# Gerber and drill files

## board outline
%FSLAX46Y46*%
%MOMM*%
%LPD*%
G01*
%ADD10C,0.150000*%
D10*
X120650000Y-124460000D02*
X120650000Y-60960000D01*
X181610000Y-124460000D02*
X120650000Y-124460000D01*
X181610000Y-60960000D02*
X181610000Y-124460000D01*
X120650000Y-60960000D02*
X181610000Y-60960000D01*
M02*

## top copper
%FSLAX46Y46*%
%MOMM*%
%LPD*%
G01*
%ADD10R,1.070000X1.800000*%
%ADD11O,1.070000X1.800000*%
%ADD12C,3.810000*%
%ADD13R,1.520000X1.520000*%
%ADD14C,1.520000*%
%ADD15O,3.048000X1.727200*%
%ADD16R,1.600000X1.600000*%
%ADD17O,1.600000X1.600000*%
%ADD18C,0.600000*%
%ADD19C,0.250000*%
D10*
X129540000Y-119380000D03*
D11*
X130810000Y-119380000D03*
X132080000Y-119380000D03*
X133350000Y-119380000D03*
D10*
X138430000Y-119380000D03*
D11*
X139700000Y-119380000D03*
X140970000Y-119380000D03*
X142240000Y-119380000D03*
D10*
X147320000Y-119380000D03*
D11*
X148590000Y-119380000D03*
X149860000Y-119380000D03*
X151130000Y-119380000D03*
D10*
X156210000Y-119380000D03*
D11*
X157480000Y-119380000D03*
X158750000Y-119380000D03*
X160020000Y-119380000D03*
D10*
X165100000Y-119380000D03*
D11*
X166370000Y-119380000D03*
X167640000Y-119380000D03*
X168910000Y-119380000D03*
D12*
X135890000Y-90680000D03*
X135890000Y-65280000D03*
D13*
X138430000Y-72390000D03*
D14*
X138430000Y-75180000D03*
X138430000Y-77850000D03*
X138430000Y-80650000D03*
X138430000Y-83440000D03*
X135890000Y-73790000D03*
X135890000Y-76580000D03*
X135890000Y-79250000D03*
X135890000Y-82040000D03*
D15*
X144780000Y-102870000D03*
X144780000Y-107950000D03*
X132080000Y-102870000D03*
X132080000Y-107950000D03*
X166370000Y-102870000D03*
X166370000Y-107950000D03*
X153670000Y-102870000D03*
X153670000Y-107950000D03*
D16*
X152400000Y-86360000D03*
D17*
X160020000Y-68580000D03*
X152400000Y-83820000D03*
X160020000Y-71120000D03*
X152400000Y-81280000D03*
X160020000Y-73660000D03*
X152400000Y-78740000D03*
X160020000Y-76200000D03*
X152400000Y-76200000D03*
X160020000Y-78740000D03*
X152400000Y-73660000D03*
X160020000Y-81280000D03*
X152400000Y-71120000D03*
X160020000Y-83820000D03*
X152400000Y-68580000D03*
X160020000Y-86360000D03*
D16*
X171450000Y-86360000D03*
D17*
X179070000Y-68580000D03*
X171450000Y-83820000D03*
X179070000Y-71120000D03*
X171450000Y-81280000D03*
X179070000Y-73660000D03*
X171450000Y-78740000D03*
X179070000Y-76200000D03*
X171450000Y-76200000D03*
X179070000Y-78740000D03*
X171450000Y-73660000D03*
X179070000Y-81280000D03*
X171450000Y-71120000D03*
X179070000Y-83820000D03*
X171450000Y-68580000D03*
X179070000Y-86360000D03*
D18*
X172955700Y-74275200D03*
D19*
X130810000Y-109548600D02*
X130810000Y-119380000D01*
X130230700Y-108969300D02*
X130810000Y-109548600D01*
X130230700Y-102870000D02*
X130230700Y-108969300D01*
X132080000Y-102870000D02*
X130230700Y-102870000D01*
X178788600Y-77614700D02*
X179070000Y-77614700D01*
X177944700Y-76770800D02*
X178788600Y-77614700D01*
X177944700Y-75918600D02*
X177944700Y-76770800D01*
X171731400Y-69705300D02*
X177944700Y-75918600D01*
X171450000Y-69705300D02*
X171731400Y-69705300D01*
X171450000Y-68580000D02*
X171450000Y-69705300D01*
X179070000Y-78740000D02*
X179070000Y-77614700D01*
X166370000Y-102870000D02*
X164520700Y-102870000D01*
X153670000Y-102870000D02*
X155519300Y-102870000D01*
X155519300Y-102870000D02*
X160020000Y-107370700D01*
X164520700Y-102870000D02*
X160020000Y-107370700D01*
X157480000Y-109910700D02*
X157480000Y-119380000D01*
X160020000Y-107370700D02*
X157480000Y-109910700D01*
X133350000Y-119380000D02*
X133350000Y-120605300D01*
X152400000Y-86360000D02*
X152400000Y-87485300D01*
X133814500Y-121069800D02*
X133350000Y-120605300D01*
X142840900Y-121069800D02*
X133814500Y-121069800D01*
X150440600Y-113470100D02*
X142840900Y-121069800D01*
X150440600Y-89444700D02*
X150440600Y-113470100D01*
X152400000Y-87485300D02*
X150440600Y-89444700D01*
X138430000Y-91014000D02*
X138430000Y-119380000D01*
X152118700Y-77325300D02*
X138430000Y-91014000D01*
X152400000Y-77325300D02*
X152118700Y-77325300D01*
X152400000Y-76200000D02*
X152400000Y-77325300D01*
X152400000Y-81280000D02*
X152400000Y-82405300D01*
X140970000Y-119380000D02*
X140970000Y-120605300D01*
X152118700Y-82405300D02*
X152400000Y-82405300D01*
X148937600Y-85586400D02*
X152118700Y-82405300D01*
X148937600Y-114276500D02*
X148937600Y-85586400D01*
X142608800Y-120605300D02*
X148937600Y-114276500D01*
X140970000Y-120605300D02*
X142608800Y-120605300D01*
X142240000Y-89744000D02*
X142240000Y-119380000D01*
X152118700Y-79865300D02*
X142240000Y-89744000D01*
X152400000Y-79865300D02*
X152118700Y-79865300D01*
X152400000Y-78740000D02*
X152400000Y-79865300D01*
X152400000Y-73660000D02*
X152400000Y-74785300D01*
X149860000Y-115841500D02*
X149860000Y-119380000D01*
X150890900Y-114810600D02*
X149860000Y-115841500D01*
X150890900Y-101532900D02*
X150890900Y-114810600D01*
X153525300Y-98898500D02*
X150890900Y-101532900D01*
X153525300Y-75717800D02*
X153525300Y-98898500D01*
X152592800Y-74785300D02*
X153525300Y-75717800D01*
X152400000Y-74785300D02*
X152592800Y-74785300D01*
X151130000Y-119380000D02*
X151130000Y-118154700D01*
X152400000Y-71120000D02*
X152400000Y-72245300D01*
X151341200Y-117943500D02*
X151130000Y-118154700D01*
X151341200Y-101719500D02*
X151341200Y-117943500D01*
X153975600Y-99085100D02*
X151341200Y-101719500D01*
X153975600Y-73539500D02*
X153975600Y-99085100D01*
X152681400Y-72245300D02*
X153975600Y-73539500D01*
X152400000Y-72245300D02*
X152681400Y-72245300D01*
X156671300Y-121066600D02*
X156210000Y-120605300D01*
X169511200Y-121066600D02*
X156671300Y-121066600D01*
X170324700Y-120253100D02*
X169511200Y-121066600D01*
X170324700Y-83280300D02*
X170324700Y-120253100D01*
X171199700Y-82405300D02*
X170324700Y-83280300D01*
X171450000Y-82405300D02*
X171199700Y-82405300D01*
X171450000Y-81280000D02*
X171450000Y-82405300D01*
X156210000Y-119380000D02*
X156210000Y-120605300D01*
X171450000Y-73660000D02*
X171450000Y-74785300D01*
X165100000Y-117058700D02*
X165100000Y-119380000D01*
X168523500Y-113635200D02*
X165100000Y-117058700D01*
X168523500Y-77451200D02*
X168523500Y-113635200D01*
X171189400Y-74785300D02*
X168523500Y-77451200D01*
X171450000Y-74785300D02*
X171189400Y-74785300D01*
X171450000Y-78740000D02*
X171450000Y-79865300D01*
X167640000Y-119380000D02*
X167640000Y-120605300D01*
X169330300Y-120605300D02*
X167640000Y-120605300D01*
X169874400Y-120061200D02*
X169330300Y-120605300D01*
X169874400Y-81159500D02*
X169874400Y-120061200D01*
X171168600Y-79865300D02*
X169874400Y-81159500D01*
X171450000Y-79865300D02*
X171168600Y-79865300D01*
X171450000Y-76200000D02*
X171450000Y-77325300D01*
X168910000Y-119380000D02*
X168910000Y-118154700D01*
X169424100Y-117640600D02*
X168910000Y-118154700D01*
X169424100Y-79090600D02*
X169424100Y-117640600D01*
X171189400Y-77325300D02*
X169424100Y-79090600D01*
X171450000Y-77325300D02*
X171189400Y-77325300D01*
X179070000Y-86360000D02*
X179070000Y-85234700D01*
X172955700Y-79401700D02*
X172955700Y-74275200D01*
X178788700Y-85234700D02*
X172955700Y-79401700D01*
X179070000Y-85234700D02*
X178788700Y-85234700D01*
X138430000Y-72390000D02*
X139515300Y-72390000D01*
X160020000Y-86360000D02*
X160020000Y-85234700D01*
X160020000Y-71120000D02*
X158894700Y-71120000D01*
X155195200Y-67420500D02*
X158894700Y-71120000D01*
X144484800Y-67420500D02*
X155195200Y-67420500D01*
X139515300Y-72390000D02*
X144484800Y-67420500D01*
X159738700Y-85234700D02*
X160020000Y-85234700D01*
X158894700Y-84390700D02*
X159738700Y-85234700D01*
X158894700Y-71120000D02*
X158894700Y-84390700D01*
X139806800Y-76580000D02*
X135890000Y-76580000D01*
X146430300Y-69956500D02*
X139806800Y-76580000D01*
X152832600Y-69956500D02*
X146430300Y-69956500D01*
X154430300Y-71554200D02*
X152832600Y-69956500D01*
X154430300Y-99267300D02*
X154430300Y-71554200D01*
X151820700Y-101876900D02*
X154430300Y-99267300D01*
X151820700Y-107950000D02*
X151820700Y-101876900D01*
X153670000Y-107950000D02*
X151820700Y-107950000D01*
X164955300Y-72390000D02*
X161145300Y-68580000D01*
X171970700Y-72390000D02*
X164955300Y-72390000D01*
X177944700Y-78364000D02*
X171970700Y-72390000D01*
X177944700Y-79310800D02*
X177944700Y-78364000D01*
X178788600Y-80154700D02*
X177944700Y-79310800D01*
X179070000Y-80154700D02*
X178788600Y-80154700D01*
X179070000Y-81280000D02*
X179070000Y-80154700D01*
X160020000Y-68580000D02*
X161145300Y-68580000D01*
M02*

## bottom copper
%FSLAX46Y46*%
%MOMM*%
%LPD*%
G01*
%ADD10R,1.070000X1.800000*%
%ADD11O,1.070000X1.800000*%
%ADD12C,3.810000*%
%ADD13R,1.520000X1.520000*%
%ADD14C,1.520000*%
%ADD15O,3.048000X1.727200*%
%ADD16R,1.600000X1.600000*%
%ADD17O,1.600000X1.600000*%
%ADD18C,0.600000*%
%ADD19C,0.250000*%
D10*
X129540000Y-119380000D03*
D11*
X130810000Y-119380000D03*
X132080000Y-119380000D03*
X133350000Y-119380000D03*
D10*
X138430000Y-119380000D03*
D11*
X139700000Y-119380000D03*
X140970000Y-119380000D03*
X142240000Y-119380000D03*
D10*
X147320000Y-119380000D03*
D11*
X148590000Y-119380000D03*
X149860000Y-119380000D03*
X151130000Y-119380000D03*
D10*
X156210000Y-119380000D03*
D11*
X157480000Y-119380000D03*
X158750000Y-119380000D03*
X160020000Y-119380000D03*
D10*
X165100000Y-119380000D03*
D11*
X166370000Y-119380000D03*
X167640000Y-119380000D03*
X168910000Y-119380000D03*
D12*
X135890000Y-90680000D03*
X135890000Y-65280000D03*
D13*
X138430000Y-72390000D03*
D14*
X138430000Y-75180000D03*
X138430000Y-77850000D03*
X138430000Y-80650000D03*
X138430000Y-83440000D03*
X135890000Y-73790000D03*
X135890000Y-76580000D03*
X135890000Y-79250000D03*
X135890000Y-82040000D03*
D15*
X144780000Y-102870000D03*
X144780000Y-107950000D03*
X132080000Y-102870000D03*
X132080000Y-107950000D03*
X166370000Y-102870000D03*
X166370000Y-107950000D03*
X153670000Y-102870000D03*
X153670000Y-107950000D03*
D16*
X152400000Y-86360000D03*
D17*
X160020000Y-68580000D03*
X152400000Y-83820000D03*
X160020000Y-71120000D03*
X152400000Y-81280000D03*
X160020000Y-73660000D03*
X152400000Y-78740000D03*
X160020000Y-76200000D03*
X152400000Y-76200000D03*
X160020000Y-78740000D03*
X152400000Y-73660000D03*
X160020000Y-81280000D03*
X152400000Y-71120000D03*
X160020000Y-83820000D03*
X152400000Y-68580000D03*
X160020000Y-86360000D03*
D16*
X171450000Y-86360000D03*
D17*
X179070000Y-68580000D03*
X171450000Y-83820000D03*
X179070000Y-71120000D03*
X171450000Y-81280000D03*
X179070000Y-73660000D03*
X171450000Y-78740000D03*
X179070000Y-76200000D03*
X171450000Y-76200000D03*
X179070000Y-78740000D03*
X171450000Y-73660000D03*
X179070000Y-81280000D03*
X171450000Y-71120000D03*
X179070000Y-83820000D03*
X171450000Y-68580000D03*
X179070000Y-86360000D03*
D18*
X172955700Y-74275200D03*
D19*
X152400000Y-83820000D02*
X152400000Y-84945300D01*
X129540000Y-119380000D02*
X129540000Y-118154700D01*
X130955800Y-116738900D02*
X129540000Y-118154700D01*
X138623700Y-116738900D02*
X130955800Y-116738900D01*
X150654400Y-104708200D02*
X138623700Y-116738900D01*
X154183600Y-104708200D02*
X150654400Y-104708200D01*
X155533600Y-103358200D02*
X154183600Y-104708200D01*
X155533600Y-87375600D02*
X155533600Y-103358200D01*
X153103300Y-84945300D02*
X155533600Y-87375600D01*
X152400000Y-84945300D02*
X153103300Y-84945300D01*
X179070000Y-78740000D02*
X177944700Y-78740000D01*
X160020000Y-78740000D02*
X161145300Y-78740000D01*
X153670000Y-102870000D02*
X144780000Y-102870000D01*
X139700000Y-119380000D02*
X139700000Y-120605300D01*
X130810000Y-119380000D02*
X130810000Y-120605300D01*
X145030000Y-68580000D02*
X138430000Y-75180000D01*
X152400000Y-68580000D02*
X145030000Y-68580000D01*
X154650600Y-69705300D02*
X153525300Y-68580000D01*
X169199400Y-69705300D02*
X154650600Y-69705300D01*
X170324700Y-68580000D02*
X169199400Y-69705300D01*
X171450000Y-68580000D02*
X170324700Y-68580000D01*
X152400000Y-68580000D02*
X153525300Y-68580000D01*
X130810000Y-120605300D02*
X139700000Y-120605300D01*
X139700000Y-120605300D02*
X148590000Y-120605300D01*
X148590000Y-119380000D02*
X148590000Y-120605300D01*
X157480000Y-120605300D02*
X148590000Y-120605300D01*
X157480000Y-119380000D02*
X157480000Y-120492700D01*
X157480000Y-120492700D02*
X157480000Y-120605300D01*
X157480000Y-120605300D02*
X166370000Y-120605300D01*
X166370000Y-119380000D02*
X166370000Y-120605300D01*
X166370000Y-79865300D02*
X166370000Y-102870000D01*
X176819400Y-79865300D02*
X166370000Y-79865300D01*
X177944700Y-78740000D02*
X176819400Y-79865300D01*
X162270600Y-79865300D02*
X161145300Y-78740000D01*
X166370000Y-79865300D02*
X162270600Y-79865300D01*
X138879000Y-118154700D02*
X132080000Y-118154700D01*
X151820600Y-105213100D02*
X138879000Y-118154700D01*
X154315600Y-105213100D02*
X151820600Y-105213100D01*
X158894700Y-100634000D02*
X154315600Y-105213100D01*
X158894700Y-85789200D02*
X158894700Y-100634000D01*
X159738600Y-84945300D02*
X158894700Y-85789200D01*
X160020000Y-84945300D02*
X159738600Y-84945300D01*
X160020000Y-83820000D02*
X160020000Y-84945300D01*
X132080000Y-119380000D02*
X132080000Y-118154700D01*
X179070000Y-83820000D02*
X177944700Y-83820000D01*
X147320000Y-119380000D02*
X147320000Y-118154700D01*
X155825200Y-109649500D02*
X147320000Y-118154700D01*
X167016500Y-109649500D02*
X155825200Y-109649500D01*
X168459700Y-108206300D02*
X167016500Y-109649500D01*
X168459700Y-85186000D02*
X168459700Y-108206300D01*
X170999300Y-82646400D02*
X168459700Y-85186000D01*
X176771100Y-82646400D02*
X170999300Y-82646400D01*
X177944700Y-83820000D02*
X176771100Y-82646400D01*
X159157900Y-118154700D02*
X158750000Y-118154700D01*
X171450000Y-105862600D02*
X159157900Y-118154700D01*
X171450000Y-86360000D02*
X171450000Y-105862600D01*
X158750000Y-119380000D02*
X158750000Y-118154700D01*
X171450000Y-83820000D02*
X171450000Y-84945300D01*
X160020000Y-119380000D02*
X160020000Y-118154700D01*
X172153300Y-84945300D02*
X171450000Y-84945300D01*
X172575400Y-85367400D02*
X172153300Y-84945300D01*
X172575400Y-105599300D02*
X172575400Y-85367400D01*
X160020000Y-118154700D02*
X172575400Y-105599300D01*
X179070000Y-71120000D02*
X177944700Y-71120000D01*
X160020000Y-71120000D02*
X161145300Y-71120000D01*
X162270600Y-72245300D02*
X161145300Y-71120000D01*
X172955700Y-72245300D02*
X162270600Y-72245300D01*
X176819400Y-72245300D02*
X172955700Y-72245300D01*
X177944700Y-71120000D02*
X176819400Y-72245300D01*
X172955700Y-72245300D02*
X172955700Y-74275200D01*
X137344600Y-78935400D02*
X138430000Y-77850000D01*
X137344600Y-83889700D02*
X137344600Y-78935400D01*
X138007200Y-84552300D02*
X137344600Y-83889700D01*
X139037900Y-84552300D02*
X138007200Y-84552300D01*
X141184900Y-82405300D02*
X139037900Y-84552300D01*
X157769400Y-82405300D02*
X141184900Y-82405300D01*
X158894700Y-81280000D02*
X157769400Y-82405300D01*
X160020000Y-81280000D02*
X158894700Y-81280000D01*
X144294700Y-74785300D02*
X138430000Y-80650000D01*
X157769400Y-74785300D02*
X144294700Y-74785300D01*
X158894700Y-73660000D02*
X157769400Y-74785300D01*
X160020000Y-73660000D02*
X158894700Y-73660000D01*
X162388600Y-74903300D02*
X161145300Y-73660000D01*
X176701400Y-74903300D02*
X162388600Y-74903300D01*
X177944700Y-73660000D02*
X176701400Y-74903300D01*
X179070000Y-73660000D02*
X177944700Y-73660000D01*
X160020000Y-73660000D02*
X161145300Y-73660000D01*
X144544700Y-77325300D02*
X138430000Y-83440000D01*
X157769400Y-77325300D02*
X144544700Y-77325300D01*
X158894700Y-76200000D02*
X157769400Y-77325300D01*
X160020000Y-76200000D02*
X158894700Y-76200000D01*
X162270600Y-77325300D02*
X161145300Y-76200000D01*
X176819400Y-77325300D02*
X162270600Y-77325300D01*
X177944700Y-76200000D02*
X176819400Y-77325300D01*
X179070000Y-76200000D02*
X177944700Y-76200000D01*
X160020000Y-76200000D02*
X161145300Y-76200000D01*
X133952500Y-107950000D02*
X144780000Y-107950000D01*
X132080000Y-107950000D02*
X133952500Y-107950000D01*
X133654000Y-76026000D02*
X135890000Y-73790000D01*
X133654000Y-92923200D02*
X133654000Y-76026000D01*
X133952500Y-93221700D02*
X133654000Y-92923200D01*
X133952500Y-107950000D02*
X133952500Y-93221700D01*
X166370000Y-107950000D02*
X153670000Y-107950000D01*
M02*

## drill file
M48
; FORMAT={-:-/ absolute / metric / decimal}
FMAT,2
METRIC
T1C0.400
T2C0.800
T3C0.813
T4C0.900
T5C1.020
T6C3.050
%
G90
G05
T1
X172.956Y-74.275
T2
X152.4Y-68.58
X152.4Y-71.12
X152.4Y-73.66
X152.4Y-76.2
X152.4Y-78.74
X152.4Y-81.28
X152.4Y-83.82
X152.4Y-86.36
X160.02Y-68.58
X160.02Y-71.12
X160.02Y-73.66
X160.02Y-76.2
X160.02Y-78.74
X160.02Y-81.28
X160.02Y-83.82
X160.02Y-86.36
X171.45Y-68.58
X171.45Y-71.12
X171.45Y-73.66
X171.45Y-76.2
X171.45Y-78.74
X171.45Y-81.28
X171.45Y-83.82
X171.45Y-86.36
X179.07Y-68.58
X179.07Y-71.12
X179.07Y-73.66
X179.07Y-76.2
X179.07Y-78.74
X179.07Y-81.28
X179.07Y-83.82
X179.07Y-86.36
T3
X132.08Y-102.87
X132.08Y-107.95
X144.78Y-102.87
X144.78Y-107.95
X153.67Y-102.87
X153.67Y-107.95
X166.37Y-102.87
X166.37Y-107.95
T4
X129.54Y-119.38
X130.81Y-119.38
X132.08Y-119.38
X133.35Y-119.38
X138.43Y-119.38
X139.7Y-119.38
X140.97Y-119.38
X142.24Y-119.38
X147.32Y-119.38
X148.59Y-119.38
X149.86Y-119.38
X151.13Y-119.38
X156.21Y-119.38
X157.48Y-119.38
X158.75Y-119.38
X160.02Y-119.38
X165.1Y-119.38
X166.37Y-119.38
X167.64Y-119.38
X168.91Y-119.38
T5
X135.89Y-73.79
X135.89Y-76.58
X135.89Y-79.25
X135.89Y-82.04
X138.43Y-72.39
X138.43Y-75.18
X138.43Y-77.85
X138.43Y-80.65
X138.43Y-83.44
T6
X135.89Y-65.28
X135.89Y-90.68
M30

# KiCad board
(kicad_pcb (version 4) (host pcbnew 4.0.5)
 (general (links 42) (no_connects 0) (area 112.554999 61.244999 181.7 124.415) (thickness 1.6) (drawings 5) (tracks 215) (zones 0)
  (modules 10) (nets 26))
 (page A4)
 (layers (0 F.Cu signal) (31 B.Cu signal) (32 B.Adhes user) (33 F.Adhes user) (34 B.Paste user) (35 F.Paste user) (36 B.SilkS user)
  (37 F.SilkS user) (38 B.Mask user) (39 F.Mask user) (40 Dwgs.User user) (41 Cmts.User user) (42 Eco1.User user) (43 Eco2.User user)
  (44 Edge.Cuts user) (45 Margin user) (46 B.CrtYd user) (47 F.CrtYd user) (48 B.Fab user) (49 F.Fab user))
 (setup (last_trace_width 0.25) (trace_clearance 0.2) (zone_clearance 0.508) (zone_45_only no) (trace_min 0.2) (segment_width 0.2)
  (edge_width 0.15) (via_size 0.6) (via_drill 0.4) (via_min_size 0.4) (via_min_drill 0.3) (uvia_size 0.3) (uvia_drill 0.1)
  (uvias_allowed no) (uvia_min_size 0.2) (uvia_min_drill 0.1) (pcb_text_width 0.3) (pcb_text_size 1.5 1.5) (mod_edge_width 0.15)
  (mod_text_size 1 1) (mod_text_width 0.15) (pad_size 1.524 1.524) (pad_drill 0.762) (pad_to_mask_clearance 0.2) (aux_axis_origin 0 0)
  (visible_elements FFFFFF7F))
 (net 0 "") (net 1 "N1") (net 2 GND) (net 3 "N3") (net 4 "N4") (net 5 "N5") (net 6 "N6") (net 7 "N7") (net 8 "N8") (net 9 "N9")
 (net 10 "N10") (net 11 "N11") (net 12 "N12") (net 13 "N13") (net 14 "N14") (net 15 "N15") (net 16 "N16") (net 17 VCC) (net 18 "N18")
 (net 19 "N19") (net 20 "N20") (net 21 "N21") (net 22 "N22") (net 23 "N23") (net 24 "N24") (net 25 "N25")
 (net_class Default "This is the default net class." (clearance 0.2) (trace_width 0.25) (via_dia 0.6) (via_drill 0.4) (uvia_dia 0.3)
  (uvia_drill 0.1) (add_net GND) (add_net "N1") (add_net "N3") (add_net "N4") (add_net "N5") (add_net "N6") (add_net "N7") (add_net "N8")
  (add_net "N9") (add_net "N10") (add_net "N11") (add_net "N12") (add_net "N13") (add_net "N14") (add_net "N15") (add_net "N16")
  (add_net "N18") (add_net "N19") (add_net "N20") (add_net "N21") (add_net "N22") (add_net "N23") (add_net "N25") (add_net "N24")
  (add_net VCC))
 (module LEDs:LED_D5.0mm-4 (layer F.Cu) (at 129.54 119.38)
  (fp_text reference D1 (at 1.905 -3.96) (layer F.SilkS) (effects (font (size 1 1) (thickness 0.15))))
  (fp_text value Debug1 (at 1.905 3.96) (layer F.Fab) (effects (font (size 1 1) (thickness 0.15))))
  (pad 1 thru_hole rect (at 0 0) (size 1.07 1.8) (drill 0.9) (layers *.Cu *.Mask) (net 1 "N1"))
  (pad 2 thru_hole oval (at 1.27 0) (size 1.07 1.8) (drill 0.9) (layers *.Cu *.Mask) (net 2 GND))
  (pad 3 thru_hole oval (at 2.54 0) (size 1.07 1.8) (drill 0.9) (layers *.Cu *.Mask) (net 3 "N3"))
  (pad 4 thru_hole oval (at 3.81 0) (size 1.07 1.8) (drill 0.9) (layers *.Cu *.Mask) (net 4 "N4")))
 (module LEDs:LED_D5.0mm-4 (layer F.Cu) (at 138.43 119.38)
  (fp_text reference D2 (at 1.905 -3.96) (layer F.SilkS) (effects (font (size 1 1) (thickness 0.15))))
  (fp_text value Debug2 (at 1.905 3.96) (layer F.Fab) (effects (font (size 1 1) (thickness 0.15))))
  (pad 1 thru_hole rect (at 0 0) (size 1.07 1.8) (drill 0.9) (layers *.Cu *.Mask) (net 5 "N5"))
  (pad 2 thru_hole oval (at 1.27 0) (size 1.07 1.8) (drill 0.9) (layers *.Cu *.Mask) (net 2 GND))
  (pad 3 thru_hole oval (at 2.54 0) (size 1.07 1.8) (drill 0.9) (layers *.Cu *.Mask) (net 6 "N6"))
  (pad 4 thru_hole oval (at 3.81 0) (size 1.07 1.8) (drill 0.9) (layers *.Cu *.Mask) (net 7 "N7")))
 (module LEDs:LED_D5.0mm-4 (layer F.Cu) (at 147.32 119.38)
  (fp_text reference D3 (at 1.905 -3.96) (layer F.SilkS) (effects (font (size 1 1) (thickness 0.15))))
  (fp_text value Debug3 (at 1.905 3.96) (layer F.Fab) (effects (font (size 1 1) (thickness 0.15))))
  (pad 1 thru_hole rect (at 0 0) (size 1.07 1.8) (drill 0.9) (layers *.Cu *.Mask) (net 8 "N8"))
  (pad 2 thru_hole oval (at 1.27 0) (size 1.07 1.8) (drill 0.9) (layers *.Cu *.Mask) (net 2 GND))
  (pad 3 thru_hole oval (at 2.54 0) (size 1.07 1.8) (drill 0.9) (layers *.Cu *.Mask) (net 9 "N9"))
  (pad 4 thru_hole oval (at 3.81 0) (size 1.07 1.8) (drill 0.9) (layers *.Cu *.Mask) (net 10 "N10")))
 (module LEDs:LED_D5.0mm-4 (layer F.Cu) (at 156.21 119.38)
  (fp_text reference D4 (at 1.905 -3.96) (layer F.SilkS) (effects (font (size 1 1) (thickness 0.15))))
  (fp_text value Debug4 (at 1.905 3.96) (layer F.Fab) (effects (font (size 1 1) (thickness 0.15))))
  (pad 1 thru_hole rect (at 0 0) (size 1.07 1.8) (drill 0.9) (layers *.Cu *.Mask) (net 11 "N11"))
  (pad 2 thru_hole oval (at 1.27 0) (size 1.07 1.8) (drill 0.9) (layers *.Cu *.Mask) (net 2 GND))
  (pad 3 thru_hole oval (at 2.54 0) (size 1.07 1.8) (drill 0.9) (layers *.Cu *.Mask) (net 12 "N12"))
  (pad 4 thru_hole oval (at 3.81 0) (size 1.07 1.8) (drill 0.9) (layers *.Cu *.Mask) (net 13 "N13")))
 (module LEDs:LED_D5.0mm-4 (layer F.Cu) (at 165.1 119.38)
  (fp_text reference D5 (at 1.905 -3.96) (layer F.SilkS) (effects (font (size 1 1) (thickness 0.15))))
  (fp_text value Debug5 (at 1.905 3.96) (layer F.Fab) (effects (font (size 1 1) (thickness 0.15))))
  (pad 1 thru_hole rect (at 0 0) (size 1.07 1.8) (drill 0.9) (layers *.Cu *.Mask) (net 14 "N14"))
  (pad 2 thru_hole oval (at 1.27 0) (size 1.07 1.8) (drill 0.9) (layers *.Cu *.Mask) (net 2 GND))
  (pad 3 thru_hole oval (at 2.54 0) (size 1.07 1.8) (drill 0.9) (layers *.Cu *.Mask) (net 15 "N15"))
  (pad 4 thru_hole oval (at 3.81 0) (size 1.07 1.8) (drill 0.9) (layers *.Cu *.Mask) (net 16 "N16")))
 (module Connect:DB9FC (layer B.Cu) (at 138.43 72.39 270)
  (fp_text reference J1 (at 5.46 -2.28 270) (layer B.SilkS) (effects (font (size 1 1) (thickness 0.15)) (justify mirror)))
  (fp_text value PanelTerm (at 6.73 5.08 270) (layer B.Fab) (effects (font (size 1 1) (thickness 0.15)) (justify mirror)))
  (pad "" thru_hole circle (at 18.29 2.54 270) (size 3.81 3.81) (drill 3.05) (layers *.Cu *.Mask))
  (pad "" thru_hole circle (at -7.11 2.54 270) (size 3.81 3.81) (drill 3.05) (layers *.Cu *.Mask))
  (pad 1 thru_hole rect (at 0 0 270) (size 1.52 1.52) (drill 1.02) (layers *.Cu *.Mask) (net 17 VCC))
  (pad 2 thru_hole circle (at 2.79 0 270) (size 1.52 1.52) (drill 1.02) (layers *.Cu *.Mask) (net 2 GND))
  (pad 3 thru_hole circle (at 5.46 0 270) (size 1.52 1.52) (drill 1.02) (layers *.Cu *.Mask) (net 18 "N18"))
  (pad 4 thru_hole circle (at 8.26 0 270) (size 1.52 1.52) (drill 1.02) (layers *.Cu *.Mask) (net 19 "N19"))
  (pad 5 thru_hole circle (at 11.05 0 270) (size 1.52 1.52) (drill 1.02) (layers *.Cu *.Mask) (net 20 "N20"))
  (pad 6 thru_hole circle (at 1.4 2.54 270) (size 1.52 1.52) (drill 1.02) (layers *.Cu *.Mask) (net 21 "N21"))
  (pad 7 thru_hole circle (at 4.19 2.54 270) (size 1.52 1.52) (drill 1.02) (layers *.Cu *.Mask) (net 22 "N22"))
  (pad 8 thru_hole circle (at 6.86 2.54 270) (size 1.52 1.52) (drill 1.02) (layers *.Cu *.Mask))
  (pad 9 thru_hole circle (at 9.65 2.54 270) (size 1.52 1.52) (drill 1.02) (layers *.Cu *.Mask)))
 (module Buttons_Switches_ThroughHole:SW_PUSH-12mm (layer F.Cu) (at 138.43 105.41)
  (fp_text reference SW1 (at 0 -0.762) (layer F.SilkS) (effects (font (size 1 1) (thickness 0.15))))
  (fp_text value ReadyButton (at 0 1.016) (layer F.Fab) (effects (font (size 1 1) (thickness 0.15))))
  (pad 1 thru_hole oval (at 6.35 -2.54) (size 3.048 1.7272) (drill 0.8128) (layers *.Cu *.Mask) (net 2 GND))
  (pad 2 thru_hole oval (at 6.35 2.54) (size 3.048 1.7272) (drill 0.8128) (layers *.Cu *.Mask) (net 21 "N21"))
  (pad 1 thru_hole oval (at -6.35 -2.54) (size 3.048 1.7272) (drill 0.8128) (layers *.Cu *.Mask) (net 2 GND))
  (pad 2 thru_hole oval (at -6.35 2.54) (size 3.048 1.7272) (drill 0.8128) (layers *.Cu *.Mask) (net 21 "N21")))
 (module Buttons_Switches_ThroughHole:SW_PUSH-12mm (layer F.Cu) (at 160.02 105.41)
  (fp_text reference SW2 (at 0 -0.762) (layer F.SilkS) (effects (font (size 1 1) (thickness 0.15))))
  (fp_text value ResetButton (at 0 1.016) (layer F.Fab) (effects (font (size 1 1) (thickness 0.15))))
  (pad 1 thru_hole oval (at 6.35 -2.54) (size 3.048 1.7272) (drill 0.8128) (layers *.Cu *.Mask) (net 2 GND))
  (pad 2 thru_hole oval (at 6.35 2.54) (size 3.048 1.7272) (drill 0.8128) (layers *.Cu *.Mask) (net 22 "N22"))
  (pad 1 thru_hole oval (at -6.35 -2.54) (size 3.048 1.7272) (drill 0.8128) (layers *.Cu *.Mask) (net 2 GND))
  (pad 2 thru_hole oval (at -6.35 2.54) (size 3.048 1.7272) (drill 0.8128) (layers *.Cu *.Mask) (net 22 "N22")))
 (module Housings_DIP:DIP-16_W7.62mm (layer B.Cu) (at 152.4 86.36)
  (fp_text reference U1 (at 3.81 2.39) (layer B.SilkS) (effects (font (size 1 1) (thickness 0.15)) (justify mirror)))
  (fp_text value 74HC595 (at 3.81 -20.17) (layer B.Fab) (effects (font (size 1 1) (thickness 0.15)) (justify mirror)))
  (pad 1 thru_hole rect (at 0 0) (size 1.6 1.6) (drill 0.8) (layers *.Cu *.Mask) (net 4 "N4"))
  (pad 9 thru_hole oval (at 7.62 -17.78) (size 1.6 1.6) (drill 0.8) (layers *.Cu *.Mask) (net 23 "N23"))
  (pad 2 thru_hole oval (at 0 -2.54) (size 1.6 1.6) (drill 0.8) (layers *.Cu *.Mask) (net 1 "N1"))
  (pad 10 thru_hole oval (at 7.62 -15.24) (size 1.6 1.6) (drill 0.8) (layers *.Cu *.Mask) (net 17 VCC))
  (pad 3 thru_hole oval (at 0 -5.08) (size 1.6 1.6) (drill 0.8) (layers *.Cu *.Mask) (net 6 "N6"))
  (pad 11 thru_hole oval (at 7.62 -12.7) (size 1.6 1.6) (drill 0.8) (layers *.Cu *.Mask) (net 19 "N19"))
  (pad 4 thru_hole oval (at 0 -7.62) (size 1.6 1.6) (drill 0.8) (layers *.Cu *.Mask) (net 7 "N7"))
  (pad 12 thru_hole oval (at 7.62 -10.16) (size 1.6 1.6) (drill 0.8) (layers *.Cu *.Mask) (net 20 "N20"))
  (pad 5 thru_hole oval (at 0 -10.16) (size 1.6 1.6) (drill 0.8) (layers *.Cu *.Mask) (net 5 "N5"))
  (pad 13 thru_hole oval (at 7.62 -7.62) (size 1.6 1.6) (drill 0.8) (layers *.Cu *.Mask) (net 2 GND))
  (pad 6 thru_hole oval (at 0 -12.7) (size 1.6 1.6) (drill 0.8) (layers *.Cu *.Mask) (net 9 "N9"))
  (pad 14 thru_hole oval (at 7.62 -5.08) (size 1.6 1.6) (drill 0.8) (layers *.Cu *.Mask) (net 18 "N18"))
  (pad 7 thru_hole oval (at 0 -15.24) (size 1.6 1.6) (drill 0.8) (layers *.Cu *.Mask) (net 10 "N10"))
  (pad 15 thru_hole oval (at 7.62 -2.54) (size 1.6 1.6) (drill 0.8) (layers *.Cu *.Mask) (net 3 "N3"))
  (pad 8 thru_hole oval (at 0 -17.78) (size 1.6 1.6) (drill 0.8) (layers *.Cu *.Mask) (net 2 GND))
  (pad 16 thru_hole oval (at 7.62 0) (size 1.6 1.6) (drill 0.8) (layers *.Cu *.Mask) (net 17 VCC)))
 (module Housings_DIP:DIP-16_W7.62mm (layer B.Cu) (at 171.45 86.36)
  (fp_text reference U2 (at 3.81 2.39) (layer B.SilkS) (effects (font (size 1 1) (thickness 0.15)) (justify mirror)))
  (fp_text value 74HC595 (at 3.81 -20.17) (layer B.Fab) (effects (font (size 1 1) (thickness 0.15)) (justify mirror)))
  (pad 1 thru_hole rect (at 0 0) (size 1.6 1.6) (drill 0.8) (layers *.Cu *.Mask) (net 12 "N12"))
  (pad 9 thru_hole oval (at 7.62 -17.78) (size 1.6 1.6) (drill 0.8) (layers *.Cu *.Mask) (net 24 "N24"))
  (pad 2 thru_hole oval (at 0 -2.54) (size 1.6 1.6) (drill 0.8) (layers *.Cu *.Mask) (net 13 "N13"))
  (pad 10 thru_hole oval (at 7.62 -15.24) (size 1.6 1.6) (drill 0.8) (layers *.Cu *.Mask) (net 17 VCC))
  (pad 3 thru_hole oval (at 0 -5.08) (size 1.6 1.6) (drill 0.8) (layers *.Cu *.Mask) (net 11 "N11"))
  (pad 11 thru_hole oval (at 7.62 -12.7) (size 1.6 1.6) (drill 0.8) (layers *.Cu *.Mask) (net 19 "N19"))
  (pad 4 thru_hole oval (at 0 -7.62) (size 1.6 1.6) (drill 0.8) (layers *.Cu *.Mask) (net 15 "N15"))
  (pad 12 thru_hole oval (at 7.62 -10.16) (size 1.6 1.6) (drill 0.8) (layers *.Cu *.Mask) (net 20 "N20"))
  (pad 5 thru_hole oval (at 0 -10.16) (size 1.6 1.6) (drill 0.8) (layers *.Cu *.Mask) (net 16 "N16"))
  (pad 13 thru_hole oval (at 7.62 -7.62) (size 1.6 1.6) (drill 0.8) (layers *.Cu *.Mask) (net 2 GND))
  (pad 6 thru_hole oval (at 0 -12.7) (size 1.6 1.6) (drill 0.8) (layers *.Cu *.Mask) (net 14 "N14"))
  (pad 14 thru_hole oval (at 7.62 -5.08) (size 1.6 1.6) (drill 0.8) (layers *.Cu *.Mask) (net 23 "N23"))
  (pad 7 thru_hole oval (at 0 -15.24) (size 1.6 1.6) (drill 0.8) (layers *.Cu *.Mask) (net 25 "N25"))
  (pad 15 thru_hole oval (at 7.62 -2.54) (size 1.6 1.6) (drill 0.8) (layers *.Cu *.Mask) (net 8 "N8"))
  (pad 8 thru_hole oval (at 0 -17.78) (size 1.6 1.6) (drill 0.8) (layers *.Cu *.Mask) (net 2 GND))
  (pad 16 thru_hole oval (at 7.62 0) (size 1.6 1.6) (drill 0.8) (layers *.Cu *.Mask) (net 17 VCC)))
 (gr_line (start 120.65 124.46) (end 120.65 60.96) (angle 90) (layer Edge.Cuts) (width 0.15))
 (gr_line (start 181.61 124.46) (end 120.65 124.46) (angle 90) (layer Edge.Cuts) (width 0.15))
 (gr_line (start 181.61 60.96) (end 181.61 124.46) (angle 90) (layer Edge.Cuts) (width 0.15))
 (gr_line (start 120.65 60.96) (end 181.61 60.96) (angle 90) (layer Edge.Cuts) (width 0.15))
 (segment (start 152.4 83.82) (end 152.4 84.9453) (width 0.25) (layer B.Cu) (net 1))
 (segment (start 129.54 119.38) (end 129.54 118.1547) (width 0.25) (layer B.Cu) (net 1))
 (segment (start 130.9558 116.7389) (end 129.54 118.1547) (width 0.25) (layer B.Cu) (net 1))
 (segment (start 138.6237 116.7389) (end 130.9558 116.7389) (width 0.25) (layer B.Cu) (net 1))
 (segment (start 150.6544 104.7082) (end 138.6237 116.7389) (width 0.25) (layer B.Cu) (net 1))
 (segment (start 154.1836 104.7082) (end 150.6544 104.7082) (width 0.25) (layer B.Cu) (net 1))
 (segment (start 155.5336 103.3582) (end 154.1836 104.7082) (width 0.25) (layer B.Cu) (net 1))
 (segment (start 155.5336 87.3756) (end 155.5336 103.3582) (width 0.25) (layer B.Cu) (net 1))
 (segment (start 153.1033 84.9453) (end 155.5336 87.3756) (width 0.25) (layer B.Cu) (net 1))
 (segment (start 152.4 84.9453) (end 153.1033 84.9453) (width 0.25) (layer B.Cu) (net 1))
 (segment (start 179.07 78.74) (end 177.9447 78.74) (width 0.25) (layer B.Cu) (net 2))
 (segment (start 160.02 78.74) (end 161.1453 78.74) (width 0.25) (layer B.Cu) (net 2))
 (segment (start 153.67 102.87) (end 144.78 102.87) (width 0.25) (layer B.Cu) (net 2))
 (segment (start 130.81 109.5486) (end 130.81 119.38) (width 0.25) (layer F.Cu) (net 2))
 (segment (start 130.2307 108.9693) (end 130.81 109.5486) (width 0.25) (layer F.Cu) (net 2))
 (segment (start 130.2307 102.87) (end 130.2307 108.9693) (width 0.25) (layer F.Cu) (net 2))
 (segment (start 132.08 102.87) (end 130.2307 102.87) (width 0.25) (layer F.Cu) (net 2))
 (segment (start 139.7 119.38) (end 139.7 120.6053) (width 0.25) (layer B.Cu) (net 2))
 (segment (start 130.81 119.38) (end 130.81 120.6053) (width 0.25) (layer B.Cu) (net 2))
 (segment (start 145.03 68.58) (end 138.43 75.18) (width 0.25) (layer B.Cu) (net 2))
 (segment (start 152.4 68.58) (end 145.03 68.58) (width 0.25) (layer B.Cu) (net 2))
 (segment (start 154.6506 69.7053) (end 153.5253 68.58) (width 0.25) (layer B.Cu) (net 2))
 (segment (start 169.1994 69.7053) (end 154.6506 69.7053) (width 0.25) (layer B.Cu) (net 2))
 (segment (start 170.3247 68.58) (end 169.1994 69.7053) (width 0.25) (layer B.Cu) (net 2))
 (segment (start 171.45 68.58) (end 170.3247 68.58) (width 0.25) (layer B.Cu) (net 2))
 (segment (start 152.4 68.58) (end 153.5253 68.58) (width 0.25) (layer B.Cu) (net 2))
 (segment (start 130.81 120.6053) (end 139.7 120.6053) (width 0.25) (layer B.Cu) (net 2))
 (segment (start 139.7 120.6053) (end 148.59 120.6053) (width 0.25) (layer B.Cu) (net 2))
 (segment (start 148.59 119.38) (end 148.59 120.6053) (width 0.25) (layer B.Cu) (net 2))
 (segment (start 178.7886 77.6147) (end 179.07 77.6147) (width 0.25) (layer F.Cu) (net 2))
 (segment (start 177.9447 76.7708) (end 178.7886 77.6147) (width 0.25) (layer F.Cu) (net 2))
 (segment (start 177.9447 75.9186) (end 177.9447 76.7708) (width 0.25) (layer F.Cu) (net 2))
 (segment (start 171.7314 69.7053) (end 177.9447 75.9186) (width 0.25) (layer F.Cu) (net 2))
 (segment (start 171.45 69.7053) (end 171.7314 69.7053) (width 0.25) (layer F.Cu) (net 2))
 (segment (start 171.45 68.58) (end 171.45 69.7053) (width 0.25) (layer F.Cu) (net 2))
 (segment (start 179.07 78.74) (end 179.07 77.6147) (width 0.25) (layer F.Cu) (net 2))
 (segment (start 157.48 120.6053) (end 148.59 120.6053) (width 0.25) (layer B.Cu) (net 2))
 (segment (start 157.48 119.38) (end 157.48 120.4927) (width 0.25) (layer B.Cu) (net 2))
 (segment (start 157.48 120.4927) (end 157.48 120.6053) (width 0.25) (layer B.Cu) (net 2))
 (segment (start 157.48 120.6053) (end 166.37 120.6053) (width 0.25) (layer B.Cu) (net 2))
 (segment (start 166.37 119.38) (end 166.37 120.6053) (width 0.25) (layer B.Cu) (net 2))
 (segment (start 166.37 79.8653) (end 166.37 102.87) (width 0.25) (layer B.Cu) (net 2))
 (segment (start 176.8194 79.8653) (end 166.37 79.8653) (width 0.25) (layer B.Cu) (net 2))
 (segment (start 177.9447 78.74) (end 176.8194 79.8653) (width 0.25) (layer B.Cu) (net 2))
 (segment (start 162.2706 79.8653) (end 161.1453 78.74) (width 0.25) (layer B.Cu) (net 2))
 (segment (start 166.37 79.8653) (end 162.2706 79.8653) (width 0.25) (layer B.Cu) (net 2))
 (segment (start 166.37 102.87) (end 164.5207 102.87) (width 0.25) (layer F.Cu) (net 2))
 (segment (start 153.67 102.87) (end 155.5193 102.87) (width 0.25) (layer F.Cu) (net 2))
 (segment (start 155.5193 102.87) (end 160.02 107.3707) (width 0.25) (layer F.Cu) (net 2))
 (segment (start 164.5207 102.87) (end 160.02 107.3707) (width 0.25) (layer F.Cu) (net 2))
 (segment (start 157.48 109.9107) (end 157.48 119.38) (width 0.25) (layer F.Cu) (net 2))
 (segment (start 160.02 107.3707) (end 157.48 109.9107) (width 0.25) (layer F.Cu) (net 2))
 (segment (start 138.879 118.1547) (end 132.08 118.1547) (width 0.25) (layer B.Cu) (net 3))
 (segment (start 151.8206 105.2131) (end 138.879 118.1547) (width 0.25) (layer B.Cu) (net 3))
 (segment (start 154.3156 105.2131) (end 151.8206 105.2131) (width 0.25) (layer B.Cu) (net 3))
 (segment (start 158.8947 100.634) (end 154.3156 105.2131) (width 0.25) (layer B.Cu) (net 3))
 (segment (start 158.8947 85.7892) (end 158.8947 100.634) (width 0.25) (layer B.Cu) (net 3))
 (segment (start 159.7386 84.9453) (end 158.8947 85.7892) (width 0.25) (layer B.Cu) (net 3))
 (segment (start 160.02 84.9453) (end 159.7386 84.9453) (width 0.25) (layer B.Cu) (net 3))
 (segment (start 160.02 83.82) (end 160.02 84.9453) (width 0.25) (layer B.Cu) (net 3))
 (segment (start 132.08 119.38) (end 132.08 118.1547) (width 0.25) (layer B.Cu) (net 3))
 (segment (start 133.35 119.38) (end 133.35 120.6053) (width 0.25) (layer F.Cu) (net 4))
 (segment (start 152.4 86.36) (end 152.4 87.4853) (width 0.25) (layer F.Cu) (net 4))
 (segment (start 133.8145 121.0698) (end 133.35 120.6053) (width 0.25) (layer F.Cu) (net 4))
 (segment (start 142.8409 121.0698) (end 133.8145 121.0698) (width 0.25) (layer F.Cu) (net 4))
 (segment (start 150.4406 113.4701) (end 142.8409 121.0698) (width 0.25) (layer F.Cu) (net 4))
 (segment (start 150.4406 89.4447) (end 150.4406 113.4701) (width 0.25) (layer F.Cu) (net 4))
 (segment (start 152.4 87.4853) (end 150.4406 89.4447) (width 0.25) (layer F.Cu) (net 4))
 (segment (start 138.43 91.014) (end 138.43 119.38) (width 0.25) (layer F.Cu) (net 5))
 (segment (start 152.1187 77.3253) (end 138.43 91.014) (width 0.25) (layer F.Cu) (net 5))
 (segment (start 152.4 77.3253) (end 152.1187 77.3253) (width 0.25) (layer F.Cu) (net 5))
 (segment (start 152.4 76.2) (end 152.4 77.3253) (width 0.25) (layer F.Cu) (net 5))
 (segment (start 152.4 81.28) (end 152.4 82.4053) (width 0.25) (layer F.Cu) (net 6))
 (segment (start 140.97 119.38) (end 140.97 120.6053) (width 0.25) (layer F.Cu) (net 6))
 (segment (start 152.1187 82.4053) (end 152.4 82.4053) (width 0.25) (layer F.Cu) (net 6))
 (segment (start 148.9376 85.5864) (end 152.1187 82.4053) (width 0.25) (layer F.Cu) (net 6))
 (segment (start 148.9376 114.2765) (end 148.9376 85.5864) (width 0.25) (layer F.Cu) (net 6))
 (segment (start 142.6088 120.6053) (end 148.9376 114.2765) (width 0.25) (layer F.Cu) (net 6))
 (segment (start 140.97 120.6053) (end 142.6088 120.6053) (width 0.25) (layer F.Cu) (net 6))
 (segment (start 142.24 89.744) (end 142.24 119.38) (width 0.25) (layer F.Cu) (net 7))
 (segment (start 152.1187 79.8653) (end 142.24 89.744) (width 0.25) (layer F.Cu) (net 7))
 (segment (start 152.4 79.8653) (end 152.1187 79.8653) (width 0.25) (layer F.Cu) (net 7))
 (segment (start 152.4 78.74) (end 152.4 79.8653) (width 0.25) (layer F.Cu) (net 7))
 (segment (start 179.07 83.82) (end 177.9447 83.82) (width 0.25) (layer B.Cu) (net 8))
 (segment (start 147.32 119.38) (end 147.32 118.1547) (width 0.25) (layer B.Cu) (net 8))
 (segment (start 155.8252 109.6495) (end 147.32 118.1547) (width 0.25) (layer B.Cu) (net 8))
 (segment (start 167.0165 109.6495) (end 155.8252 109.6495) (width 0.25) (layer B.Cu) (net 8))
 (segment (start 168.4597 108.2063) (end 167.0165 109.6495) (width 0.25) (layer B.Cu) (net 8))
 (segment (start 168.4597 85.186) (end 168.4597 108.2063) (width 0.25) (layer B.Cu) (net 8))
 (segment (start 170.9993 82.6464) (end 168.4597 85.186) (width 0.25) (layer B.Cu) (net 8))
 (segment (start 176.7711 82.6464) (end 170.9993 82.6464) (width 0.25) (layer B.Cu) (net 8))
 (segment (start 177.9447 83.82) (end 176.7711 82.6464) (width 0.25) (layer B.Cu) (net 8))
 (segment (start 152.4 73.66) (end 152.4 74.7853) (width 0.25) (layer F.Cu) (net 9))
 (segment (start 149.86 115.8415) (end 149.86 119.38) (width 0.25) (layer F.Cu) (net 9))
 (segment (start 150.8909 114.8106) (end 149.86 115.8415) (width 0.25) (layer F.Cu) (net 9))
 (segment (start 150.8909 101.5329) (end 150.8909 114.8106) (width 0.25) (layer F.Cu) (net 9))
 (segment (start 153.5253 98.8985) (end 150.8909 101.5329) (width 0.25) (layer F.Cu) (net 9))
 (segment (start 153.5253 75.7178) (end 153.5253 98.8985) (width 0.25) (layer F.Cu) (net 9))
 (segment (start 152.5928 74.7853) (end 153.5253 75.7178) (width 0.25) (layer F.Cu) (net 9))
 (segment (start 152.4 74.7853) (end 152.5928 74.7853) (width 0.25) (layer F.Cu) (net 9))
 (segment (start 151.13 119.38) (end 151.13 118.1547) (width 0.25) (layer F.Cu) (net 10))
 (segment (start 152.4 71.12) (end 152.4 72.2453) (width 0.25) (layer F.Cu) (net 10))
 (segment (start 151.3412 117.9435) (end 151.13 118.1547) (width 0.25) (layer F.Cu) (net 10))
 (segment (start 151.3412 101.7195) (end 151.3412 117.9435) (width 0.25) (layer F.Cu) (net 10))
 (segment (start 153.9756 99.0851) (end 151.3412 101.7195) (width 0.25) (layer F.Cu) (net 10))
 (segment (start 153.9756 73.5395) (end 153.9756 99.0851) (width 0.25) (layer F.Cu) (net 10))
 (segment (start 152.6814 72.2453) (end 153.9756 73.5395) (width 0.25) (layer F.Cu) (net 10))
 (segment (start 152.4 72.2453) (end 152.6814 72.2453) (width 0.25) (layer F.Cu) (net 10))
 (segment (start 156.6713 121.0666) (end 156.21 120.6053) (width 0.25) (layer F.Cu) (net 11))
 (segment (start 169.5112 121.0666) (end 156.6713 121.0666) (width 0.25) (layer F.Cu) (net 11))
 (segment (start 170.3247 120.2531) (end 169.5112 121.0666) (width 0.25) (layer F.Cu) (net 11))
 (segment (start 170.3247 83.2803) (end 170.3247 120.2531) (width 0.25) (layer F.Cu) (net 11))
 (segment (start 171.1997 82.4053) (end 170.3247 83.2803) (width 0.25) (layer F.Cu) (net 11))
 (segment (start 171.45 82.4053) (end 171.1997 82.4053) (width 0.25) (layer F.Cu) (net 11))
 (segment (start 171.45 81.28) (end 171.45 82.4053) (width 0.25) (layer F.Cu) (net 11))
 (segment (start 156.21 119.38) (end 156.21 120.6053) (width 0.25) (layer F.Cu) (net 11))
 (segment (start 159.1579 118.1547) (end 158.75 118.1547) (width 0.25) (layer B.Cu) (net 12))
 (segment (start 171.45 105.8626) (end 159.1579 118.1547) (width 0.25) (layer B.Cu) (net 12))
 (segment (start 171.45 86.36) (end 171.45 105.8626) (width 0.25) (layer B.Cu) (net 12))
 (segment (start 158.75 119.38) (end 158.75 118.1547) (width 0.25) (layer B.Cu) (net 12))
 (segment (start 171.45 83.82) (end 171.45 84.9453) (width 0.25) (layer B.Cu) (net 13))
 (segment (start 160.02 119.38) (end 160.02 118.1547) (width 0.25) (layer B.Cu) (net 13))
 (segment (start 172.1533 84.9453) (end 171.45 84.9453) (width 0.25) (layer B.Cu) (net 13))
 (segment (start 172.5754 85.3674) (end 172.1533 84.9453) (width 0.25) (layer B.Cu) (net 13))
 (segment (start 172.5754 105.5993) (end 172.5754 85.3674) (width 0.25) (layer B.Cu) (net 13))
 (segment (start 160.02 118.1547) (end 172.5754 105.5993) (width 0.25) (layer B.Cu) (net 13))
 (segment (start 171.45 73.66) (end 171.45 74.7853) (width 0.25) (layer F.Cu) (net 14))
 (segment (start 165.1 117.0587) (end 165.1 119.38) (width 0.25) (layer F.Cu) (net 14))
 (segment (start 168.5235 113.6352) (end 165.1 117.0587) (width 0.25) (layer F.Cu) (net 14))
 (segment (start 168.5235 77.4512) (end 168.5235 113.6352) (width 0.25) (layer F.Cu) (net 14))
 (segment (start 171.1894 74.7853) (end 168.5235 77.4512) (width 0.25) (layer F.Cu) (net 14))
 (segment (start 171.45 74.7853) (end 171.1894 74.7853) (width 0.25) (layer F.Cu) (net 14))
 (segment (start 171.45 78.74) (end 171.45 79.8653) (width 0.25) (layer F.Cu) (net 15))
 (segment (start 167.64 119.38) (end 167.64 120.6053) (width 0.25) (layer F.Cu) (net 15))
 (segment (start 169.3303 120.6053) (end 167.64 120.6053) (width 0.25) (layer F.Cu) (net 15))
 (segment (start 169.8744 120.0612) (end 169.3303 120.6053) (width 0.25) (layer F.Cu) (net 15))
 (segment (start 169.8744 81.1595) (end 169.8744 120.0612) (width 0.25) (layer F.Cu) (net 15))
 (segment (start 171.1686 79.8653) (end 169.8744 81.1595) (width 0.25) (layer F.Cu) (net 15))
 (segment (start 171.45 79.8653) (end 171.1686 79.8653) (width 0.25) (layer F.Cu) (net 15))
 (segment (start 171.45 76.2) (end 171.45 77.3253) (width 0.25) (layer F.Cu) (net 16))
 (segment (start 168.91 119.38) (end 168.91 118.1547) (width 0.25) (layer F.Cu) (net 16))
 (segment (start 169.4241 117.6406) (end 168.91 118.1547) (width 0.25) (layer F.Cu) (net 16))
 (segment (start 169.4241 79.0906) (end 169.4241 117.6406) (width 0.25) (layer F.Cu) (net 16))
 (segment (start 171.1894 77.3253) (end 169.4241 79.0906) (width 0.25) (layer F.Cu) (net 16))
 (segment (start 171.45 77.3253) (end 171.1894 77.3253) (width 0.25) (layer F.Cu) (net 16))
 (via (at 172.9557 74.2752) (size 0.6) (layers F.Cu B.Cu) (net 17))
 (segment (start 179.07 71.12) (end 177.9447 71.12) (width 0.25) (layer B.Cu) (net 17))
 (segment (start 179.07 86.36) (end 179.07 85.2347) (width 0.25) (layer F.Cu) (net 17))
 (segment (start 160.02 71.12) (end 161.1453 71.12) (width 0.25) (layer B.Cu) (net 17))
 (segment (start 162.2706 72.2453) (end 161.1453 71.12) (width 0.25) (layer B.Cu) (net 17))
 (segment (start 172.9557 72.2453) (end 162.2706 72.2453) (width 0.25) (layer B.Cu) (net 17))
 (segment (start 176.8194 72.2453) (end 172.9557 72.2453) (width 0.25) (layer B.Cu) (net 17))
 (segment (start 177.9447 71.12) (end 176.8194 72.2453) (width 0.25) (layer B.Cu) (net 17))
 (segment (start 172.9557 72.2453) (end 172.9557 74.2752) (width 0.25) (layer B.Cu) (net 17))
 (segment (start 172.9557 79.4017) (end 172.9557 74.2752) (width 0.25) (layer F.Cu) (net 17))
 (segment (start 178.7887 85.2347) (end 172.9557 79.4017) (width 0.25) (layer F.Cu) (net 17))
 (segment (start 179.07 85.2347) (end 178.7887 85.2347) (width 0.25) (layer F.Cu) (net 17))
 (segment (start 138.43 72.39) (end 139.5153 72.39) (width 0.25) (layer F.Cu) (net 17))
 (segment (start 160.02 86.36) (end 160.02 85.2347) (width 0.25) (layer F.Cu) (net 17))
 (segment (start 160.02 71.12) (end 158.8947 71.12) (width 0.25) (layer F.Cu) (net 17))
 (segment (start 155.1952 67.4205) (end 158.8947 71.12) (width 0.25) (layer F.Cu) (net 17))
 (segment (start 144.4848 67.4205) (end 155.1952 67.4205) (width 0.25) (layer F.Cu) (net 17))
 (segment (start 139.5153 72.39) (end 144.4848 67.4205) (width 0.25) (layer F.Cu) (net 17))
 (segment (start 159.7387 85.2347) (end 160.02 85.2347) (width 0.25) (layer F.Cu) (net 17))
 (segment (start 158.8947 84.3907) (end 159.7387 85.2347) (width 0.25) (layer F.Cu) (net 17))
 (segment (start 158.8947 71.12) (end 158.8947 84.3907) (width 0.25) (layer F.Cu) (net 17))
 (segment (start 137.3446 78.9354) (end 138.43 77.85) (width 0.25) (layer B.Cu) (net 18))
 (segment (start 137.3446 83.8897) (end 137.3446 78.9354) (width 0.25) (layer B.Cu) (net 18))
 (segment (start 138.0072 84.5523) (end 137.3446 83.8897) (width 0.25) (layer B.Cu) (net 18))
 (segment (start 139.0379 84.5523) (end 138.0072 84.5523) (width 0.25) (layer B.Cu) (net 18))
 (segment (start 141.1849 82.4053) (end 139.0379 84.5523) (width 0.25) (layer B.Cu) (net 18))
 (segment (start 157.7694 82.4053) (end 141.1849 82.4053) (width 0.25) (layer B.Cu) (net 18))
 (segment (start 158.8947 81.28) (end 157.7694 82.4053) (width 0.25) (layer B.Cu) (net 18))
 (segment (start 160.02 81.28) (end 158.8947 81.28) (width 0.25) (layer B.Cu) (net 18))
 (segment (start 144.2947 74.7853) (end 138.43 80.65) (width 0.25) (layer B.Cu) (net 19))
 (segment (start 157.7694 74.7853) (end 144.2947 74.7853) (width 0.25) (layer B.Cu) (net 19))
 (segment (start 158.8947 73.66) (end 157.7694 74.7853) (width 0.25) (layer B.Cu) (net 19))
 (segment (start 160.02 73.66) (end 158.8947 73.66) (width 0.25) (layer B.Cu) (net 19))
 (segment (start 162.3886 74.9033) (end 161.1453 73.66) (width 0.25) (layer B.Cu) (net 19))
 (segment (start 176.7014 74.9033) (end 162.3886 74.9033) (width 0.25) (layer B.Cu) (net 19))
 (segment (start 177.9447 73.66) (end 176.7014 74.9033) (width 0.25) (layer B.Cu) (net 19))
 (segment (start 179.07 73.66) (end 177.9447 73.66) (width 0.25) (layer B.Cu) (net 19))
 (segment (start 160.02 73.66) (end 161.1453 73.66) (width 0.25) (layer B.Cu) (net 19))
 (segment (start 144.5447 77.3253) (end 138.43 83.44) (width 0.25) (layer B.Cu) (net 20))
 (segment (start 157.7694 77.3253) (end 144.5447 77.3253) (width 0.25) (layer B.Cu) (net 20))
 (segment (start 158.8947 76.2) (end 157.7694 77.3253) (width 0.25) (layer B.Cu) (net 20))
 (segment (start 160.02 76.2) (end 158.8947 76.2) (width 0.25) (layer B.Cu) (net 20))
 (segment (start 162.2706 77.3253) (end 161.1453 76.2) (width 0.25) (layer B.Cu) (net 20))
 (segment (start 176.8194 77.3253) (end 162.2706 77.3253) (width 0.25) (layer B.Cu) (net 20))
 (segment (start 177.9447 76.2) (end 176.8194 77.3253) (width 0.25) (layer B.Cu) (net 20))
 (segment (start 179.07 76.2) (end 177.9447 76.2) (width 0.25) (layer B.Cu) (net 20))
 (segment (start 160.02 76.2) (end 161.1453 76.2) (width 0.25) (layer B.Cu) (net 20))
 (segment (start 133.9525 107.95) (end 144.78 107.95) (width 0.25) (layer B.Cu) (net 21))
 (segment (start 132.08 107.95) (end 133.9525 107.95) (width 0.25) (layer B.Cu) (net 21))
 (segment (start 133.654 76.026) (end 135.89 73.79) (width 0.25) (layer B.Cu) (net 21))
 (segment (start 133.654 92.9232) (end 133.654 76.026) (width 0.25) (layer B.Cu) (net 21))
 (segment (start 133.9525 93.2217) (end 133.654 92.9232) (width 0.25) (layer B.Cu) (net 21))
 (segment (start 133.9525 107.95) (end 133.9525 93.2217) (width 0.25) (layer B.Cu) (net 21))
 (segment (start 166.37 107.95) (end 153.67 107.95) (width 0.25) (layer B.Cu) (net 22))
 (segment (start 139.8068 76.58) (end 135.89 76.58) (width 0.25) (layer F.Cu) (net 22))
 (segment (start 146.4303 69.9565) (end 139.8068 76.58) (width 0.25) (layer F.Cu) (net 22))
 (segment (start 152.8326 69.9565) (end 146.4303 69.9565) (width 0.25) (layer F.Cu) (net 22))
 (segment (start 154.4303 71.5542) (end 152.8326 69.9565) (width 0.25) (layer F.Cu) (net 22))
 (segment (start 154.4303 99.2673) (end 154.4303 71.5542) (width 0.25) (layer F.Cu) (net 22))
 (segment (start 151.8207 101.8769) (end 154.4303 99.2673) (width 0.25) (layer F.Cu) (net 22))
 (segment (start 151.8207 107.95) (end 151.8207 101.8769) (width 0.25) (layer F.Cu) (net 22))
 (segment (start 153.67 107.95) (end 151.8207 107.95) (width 0.25) (layer F.Cu) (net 22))
 (segment (start 164.9553 72.39) (end 161.1453 68.58) (width 0.25) (layer F.Cu) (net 23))
 (segment (start 171.9707 72.39) (end 164.9553 72.39) (width 0.25) (layer F.Cu) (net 23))
 (segment (start 177.9447 78.364) (end 171.9707 72.39) (width 0.25) (layer F.Cu) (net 23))
 (segment (start 177.9447 79.3108) (end 177.9447 78.364) (width 0.25) (layer F.Cu) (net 23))
 (segment (start 178.7886 80.1547) (end 177.9447 79.3108) (width 0.25) (layer F.Cu) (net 23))
 (segment (start 179.07 80.1547) (end 178.7886 80.1547) (width 0.25) (layer F.Cu) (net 23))
 (segment (start 179.07 81.28) (end 179.07 80.1547) (width 0.25) (layer F.Cu) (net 23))
 (segment (start 160.02 68.58) (end 161.1453 68.58) (width 0.25) (layer F.Cu) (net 23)))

